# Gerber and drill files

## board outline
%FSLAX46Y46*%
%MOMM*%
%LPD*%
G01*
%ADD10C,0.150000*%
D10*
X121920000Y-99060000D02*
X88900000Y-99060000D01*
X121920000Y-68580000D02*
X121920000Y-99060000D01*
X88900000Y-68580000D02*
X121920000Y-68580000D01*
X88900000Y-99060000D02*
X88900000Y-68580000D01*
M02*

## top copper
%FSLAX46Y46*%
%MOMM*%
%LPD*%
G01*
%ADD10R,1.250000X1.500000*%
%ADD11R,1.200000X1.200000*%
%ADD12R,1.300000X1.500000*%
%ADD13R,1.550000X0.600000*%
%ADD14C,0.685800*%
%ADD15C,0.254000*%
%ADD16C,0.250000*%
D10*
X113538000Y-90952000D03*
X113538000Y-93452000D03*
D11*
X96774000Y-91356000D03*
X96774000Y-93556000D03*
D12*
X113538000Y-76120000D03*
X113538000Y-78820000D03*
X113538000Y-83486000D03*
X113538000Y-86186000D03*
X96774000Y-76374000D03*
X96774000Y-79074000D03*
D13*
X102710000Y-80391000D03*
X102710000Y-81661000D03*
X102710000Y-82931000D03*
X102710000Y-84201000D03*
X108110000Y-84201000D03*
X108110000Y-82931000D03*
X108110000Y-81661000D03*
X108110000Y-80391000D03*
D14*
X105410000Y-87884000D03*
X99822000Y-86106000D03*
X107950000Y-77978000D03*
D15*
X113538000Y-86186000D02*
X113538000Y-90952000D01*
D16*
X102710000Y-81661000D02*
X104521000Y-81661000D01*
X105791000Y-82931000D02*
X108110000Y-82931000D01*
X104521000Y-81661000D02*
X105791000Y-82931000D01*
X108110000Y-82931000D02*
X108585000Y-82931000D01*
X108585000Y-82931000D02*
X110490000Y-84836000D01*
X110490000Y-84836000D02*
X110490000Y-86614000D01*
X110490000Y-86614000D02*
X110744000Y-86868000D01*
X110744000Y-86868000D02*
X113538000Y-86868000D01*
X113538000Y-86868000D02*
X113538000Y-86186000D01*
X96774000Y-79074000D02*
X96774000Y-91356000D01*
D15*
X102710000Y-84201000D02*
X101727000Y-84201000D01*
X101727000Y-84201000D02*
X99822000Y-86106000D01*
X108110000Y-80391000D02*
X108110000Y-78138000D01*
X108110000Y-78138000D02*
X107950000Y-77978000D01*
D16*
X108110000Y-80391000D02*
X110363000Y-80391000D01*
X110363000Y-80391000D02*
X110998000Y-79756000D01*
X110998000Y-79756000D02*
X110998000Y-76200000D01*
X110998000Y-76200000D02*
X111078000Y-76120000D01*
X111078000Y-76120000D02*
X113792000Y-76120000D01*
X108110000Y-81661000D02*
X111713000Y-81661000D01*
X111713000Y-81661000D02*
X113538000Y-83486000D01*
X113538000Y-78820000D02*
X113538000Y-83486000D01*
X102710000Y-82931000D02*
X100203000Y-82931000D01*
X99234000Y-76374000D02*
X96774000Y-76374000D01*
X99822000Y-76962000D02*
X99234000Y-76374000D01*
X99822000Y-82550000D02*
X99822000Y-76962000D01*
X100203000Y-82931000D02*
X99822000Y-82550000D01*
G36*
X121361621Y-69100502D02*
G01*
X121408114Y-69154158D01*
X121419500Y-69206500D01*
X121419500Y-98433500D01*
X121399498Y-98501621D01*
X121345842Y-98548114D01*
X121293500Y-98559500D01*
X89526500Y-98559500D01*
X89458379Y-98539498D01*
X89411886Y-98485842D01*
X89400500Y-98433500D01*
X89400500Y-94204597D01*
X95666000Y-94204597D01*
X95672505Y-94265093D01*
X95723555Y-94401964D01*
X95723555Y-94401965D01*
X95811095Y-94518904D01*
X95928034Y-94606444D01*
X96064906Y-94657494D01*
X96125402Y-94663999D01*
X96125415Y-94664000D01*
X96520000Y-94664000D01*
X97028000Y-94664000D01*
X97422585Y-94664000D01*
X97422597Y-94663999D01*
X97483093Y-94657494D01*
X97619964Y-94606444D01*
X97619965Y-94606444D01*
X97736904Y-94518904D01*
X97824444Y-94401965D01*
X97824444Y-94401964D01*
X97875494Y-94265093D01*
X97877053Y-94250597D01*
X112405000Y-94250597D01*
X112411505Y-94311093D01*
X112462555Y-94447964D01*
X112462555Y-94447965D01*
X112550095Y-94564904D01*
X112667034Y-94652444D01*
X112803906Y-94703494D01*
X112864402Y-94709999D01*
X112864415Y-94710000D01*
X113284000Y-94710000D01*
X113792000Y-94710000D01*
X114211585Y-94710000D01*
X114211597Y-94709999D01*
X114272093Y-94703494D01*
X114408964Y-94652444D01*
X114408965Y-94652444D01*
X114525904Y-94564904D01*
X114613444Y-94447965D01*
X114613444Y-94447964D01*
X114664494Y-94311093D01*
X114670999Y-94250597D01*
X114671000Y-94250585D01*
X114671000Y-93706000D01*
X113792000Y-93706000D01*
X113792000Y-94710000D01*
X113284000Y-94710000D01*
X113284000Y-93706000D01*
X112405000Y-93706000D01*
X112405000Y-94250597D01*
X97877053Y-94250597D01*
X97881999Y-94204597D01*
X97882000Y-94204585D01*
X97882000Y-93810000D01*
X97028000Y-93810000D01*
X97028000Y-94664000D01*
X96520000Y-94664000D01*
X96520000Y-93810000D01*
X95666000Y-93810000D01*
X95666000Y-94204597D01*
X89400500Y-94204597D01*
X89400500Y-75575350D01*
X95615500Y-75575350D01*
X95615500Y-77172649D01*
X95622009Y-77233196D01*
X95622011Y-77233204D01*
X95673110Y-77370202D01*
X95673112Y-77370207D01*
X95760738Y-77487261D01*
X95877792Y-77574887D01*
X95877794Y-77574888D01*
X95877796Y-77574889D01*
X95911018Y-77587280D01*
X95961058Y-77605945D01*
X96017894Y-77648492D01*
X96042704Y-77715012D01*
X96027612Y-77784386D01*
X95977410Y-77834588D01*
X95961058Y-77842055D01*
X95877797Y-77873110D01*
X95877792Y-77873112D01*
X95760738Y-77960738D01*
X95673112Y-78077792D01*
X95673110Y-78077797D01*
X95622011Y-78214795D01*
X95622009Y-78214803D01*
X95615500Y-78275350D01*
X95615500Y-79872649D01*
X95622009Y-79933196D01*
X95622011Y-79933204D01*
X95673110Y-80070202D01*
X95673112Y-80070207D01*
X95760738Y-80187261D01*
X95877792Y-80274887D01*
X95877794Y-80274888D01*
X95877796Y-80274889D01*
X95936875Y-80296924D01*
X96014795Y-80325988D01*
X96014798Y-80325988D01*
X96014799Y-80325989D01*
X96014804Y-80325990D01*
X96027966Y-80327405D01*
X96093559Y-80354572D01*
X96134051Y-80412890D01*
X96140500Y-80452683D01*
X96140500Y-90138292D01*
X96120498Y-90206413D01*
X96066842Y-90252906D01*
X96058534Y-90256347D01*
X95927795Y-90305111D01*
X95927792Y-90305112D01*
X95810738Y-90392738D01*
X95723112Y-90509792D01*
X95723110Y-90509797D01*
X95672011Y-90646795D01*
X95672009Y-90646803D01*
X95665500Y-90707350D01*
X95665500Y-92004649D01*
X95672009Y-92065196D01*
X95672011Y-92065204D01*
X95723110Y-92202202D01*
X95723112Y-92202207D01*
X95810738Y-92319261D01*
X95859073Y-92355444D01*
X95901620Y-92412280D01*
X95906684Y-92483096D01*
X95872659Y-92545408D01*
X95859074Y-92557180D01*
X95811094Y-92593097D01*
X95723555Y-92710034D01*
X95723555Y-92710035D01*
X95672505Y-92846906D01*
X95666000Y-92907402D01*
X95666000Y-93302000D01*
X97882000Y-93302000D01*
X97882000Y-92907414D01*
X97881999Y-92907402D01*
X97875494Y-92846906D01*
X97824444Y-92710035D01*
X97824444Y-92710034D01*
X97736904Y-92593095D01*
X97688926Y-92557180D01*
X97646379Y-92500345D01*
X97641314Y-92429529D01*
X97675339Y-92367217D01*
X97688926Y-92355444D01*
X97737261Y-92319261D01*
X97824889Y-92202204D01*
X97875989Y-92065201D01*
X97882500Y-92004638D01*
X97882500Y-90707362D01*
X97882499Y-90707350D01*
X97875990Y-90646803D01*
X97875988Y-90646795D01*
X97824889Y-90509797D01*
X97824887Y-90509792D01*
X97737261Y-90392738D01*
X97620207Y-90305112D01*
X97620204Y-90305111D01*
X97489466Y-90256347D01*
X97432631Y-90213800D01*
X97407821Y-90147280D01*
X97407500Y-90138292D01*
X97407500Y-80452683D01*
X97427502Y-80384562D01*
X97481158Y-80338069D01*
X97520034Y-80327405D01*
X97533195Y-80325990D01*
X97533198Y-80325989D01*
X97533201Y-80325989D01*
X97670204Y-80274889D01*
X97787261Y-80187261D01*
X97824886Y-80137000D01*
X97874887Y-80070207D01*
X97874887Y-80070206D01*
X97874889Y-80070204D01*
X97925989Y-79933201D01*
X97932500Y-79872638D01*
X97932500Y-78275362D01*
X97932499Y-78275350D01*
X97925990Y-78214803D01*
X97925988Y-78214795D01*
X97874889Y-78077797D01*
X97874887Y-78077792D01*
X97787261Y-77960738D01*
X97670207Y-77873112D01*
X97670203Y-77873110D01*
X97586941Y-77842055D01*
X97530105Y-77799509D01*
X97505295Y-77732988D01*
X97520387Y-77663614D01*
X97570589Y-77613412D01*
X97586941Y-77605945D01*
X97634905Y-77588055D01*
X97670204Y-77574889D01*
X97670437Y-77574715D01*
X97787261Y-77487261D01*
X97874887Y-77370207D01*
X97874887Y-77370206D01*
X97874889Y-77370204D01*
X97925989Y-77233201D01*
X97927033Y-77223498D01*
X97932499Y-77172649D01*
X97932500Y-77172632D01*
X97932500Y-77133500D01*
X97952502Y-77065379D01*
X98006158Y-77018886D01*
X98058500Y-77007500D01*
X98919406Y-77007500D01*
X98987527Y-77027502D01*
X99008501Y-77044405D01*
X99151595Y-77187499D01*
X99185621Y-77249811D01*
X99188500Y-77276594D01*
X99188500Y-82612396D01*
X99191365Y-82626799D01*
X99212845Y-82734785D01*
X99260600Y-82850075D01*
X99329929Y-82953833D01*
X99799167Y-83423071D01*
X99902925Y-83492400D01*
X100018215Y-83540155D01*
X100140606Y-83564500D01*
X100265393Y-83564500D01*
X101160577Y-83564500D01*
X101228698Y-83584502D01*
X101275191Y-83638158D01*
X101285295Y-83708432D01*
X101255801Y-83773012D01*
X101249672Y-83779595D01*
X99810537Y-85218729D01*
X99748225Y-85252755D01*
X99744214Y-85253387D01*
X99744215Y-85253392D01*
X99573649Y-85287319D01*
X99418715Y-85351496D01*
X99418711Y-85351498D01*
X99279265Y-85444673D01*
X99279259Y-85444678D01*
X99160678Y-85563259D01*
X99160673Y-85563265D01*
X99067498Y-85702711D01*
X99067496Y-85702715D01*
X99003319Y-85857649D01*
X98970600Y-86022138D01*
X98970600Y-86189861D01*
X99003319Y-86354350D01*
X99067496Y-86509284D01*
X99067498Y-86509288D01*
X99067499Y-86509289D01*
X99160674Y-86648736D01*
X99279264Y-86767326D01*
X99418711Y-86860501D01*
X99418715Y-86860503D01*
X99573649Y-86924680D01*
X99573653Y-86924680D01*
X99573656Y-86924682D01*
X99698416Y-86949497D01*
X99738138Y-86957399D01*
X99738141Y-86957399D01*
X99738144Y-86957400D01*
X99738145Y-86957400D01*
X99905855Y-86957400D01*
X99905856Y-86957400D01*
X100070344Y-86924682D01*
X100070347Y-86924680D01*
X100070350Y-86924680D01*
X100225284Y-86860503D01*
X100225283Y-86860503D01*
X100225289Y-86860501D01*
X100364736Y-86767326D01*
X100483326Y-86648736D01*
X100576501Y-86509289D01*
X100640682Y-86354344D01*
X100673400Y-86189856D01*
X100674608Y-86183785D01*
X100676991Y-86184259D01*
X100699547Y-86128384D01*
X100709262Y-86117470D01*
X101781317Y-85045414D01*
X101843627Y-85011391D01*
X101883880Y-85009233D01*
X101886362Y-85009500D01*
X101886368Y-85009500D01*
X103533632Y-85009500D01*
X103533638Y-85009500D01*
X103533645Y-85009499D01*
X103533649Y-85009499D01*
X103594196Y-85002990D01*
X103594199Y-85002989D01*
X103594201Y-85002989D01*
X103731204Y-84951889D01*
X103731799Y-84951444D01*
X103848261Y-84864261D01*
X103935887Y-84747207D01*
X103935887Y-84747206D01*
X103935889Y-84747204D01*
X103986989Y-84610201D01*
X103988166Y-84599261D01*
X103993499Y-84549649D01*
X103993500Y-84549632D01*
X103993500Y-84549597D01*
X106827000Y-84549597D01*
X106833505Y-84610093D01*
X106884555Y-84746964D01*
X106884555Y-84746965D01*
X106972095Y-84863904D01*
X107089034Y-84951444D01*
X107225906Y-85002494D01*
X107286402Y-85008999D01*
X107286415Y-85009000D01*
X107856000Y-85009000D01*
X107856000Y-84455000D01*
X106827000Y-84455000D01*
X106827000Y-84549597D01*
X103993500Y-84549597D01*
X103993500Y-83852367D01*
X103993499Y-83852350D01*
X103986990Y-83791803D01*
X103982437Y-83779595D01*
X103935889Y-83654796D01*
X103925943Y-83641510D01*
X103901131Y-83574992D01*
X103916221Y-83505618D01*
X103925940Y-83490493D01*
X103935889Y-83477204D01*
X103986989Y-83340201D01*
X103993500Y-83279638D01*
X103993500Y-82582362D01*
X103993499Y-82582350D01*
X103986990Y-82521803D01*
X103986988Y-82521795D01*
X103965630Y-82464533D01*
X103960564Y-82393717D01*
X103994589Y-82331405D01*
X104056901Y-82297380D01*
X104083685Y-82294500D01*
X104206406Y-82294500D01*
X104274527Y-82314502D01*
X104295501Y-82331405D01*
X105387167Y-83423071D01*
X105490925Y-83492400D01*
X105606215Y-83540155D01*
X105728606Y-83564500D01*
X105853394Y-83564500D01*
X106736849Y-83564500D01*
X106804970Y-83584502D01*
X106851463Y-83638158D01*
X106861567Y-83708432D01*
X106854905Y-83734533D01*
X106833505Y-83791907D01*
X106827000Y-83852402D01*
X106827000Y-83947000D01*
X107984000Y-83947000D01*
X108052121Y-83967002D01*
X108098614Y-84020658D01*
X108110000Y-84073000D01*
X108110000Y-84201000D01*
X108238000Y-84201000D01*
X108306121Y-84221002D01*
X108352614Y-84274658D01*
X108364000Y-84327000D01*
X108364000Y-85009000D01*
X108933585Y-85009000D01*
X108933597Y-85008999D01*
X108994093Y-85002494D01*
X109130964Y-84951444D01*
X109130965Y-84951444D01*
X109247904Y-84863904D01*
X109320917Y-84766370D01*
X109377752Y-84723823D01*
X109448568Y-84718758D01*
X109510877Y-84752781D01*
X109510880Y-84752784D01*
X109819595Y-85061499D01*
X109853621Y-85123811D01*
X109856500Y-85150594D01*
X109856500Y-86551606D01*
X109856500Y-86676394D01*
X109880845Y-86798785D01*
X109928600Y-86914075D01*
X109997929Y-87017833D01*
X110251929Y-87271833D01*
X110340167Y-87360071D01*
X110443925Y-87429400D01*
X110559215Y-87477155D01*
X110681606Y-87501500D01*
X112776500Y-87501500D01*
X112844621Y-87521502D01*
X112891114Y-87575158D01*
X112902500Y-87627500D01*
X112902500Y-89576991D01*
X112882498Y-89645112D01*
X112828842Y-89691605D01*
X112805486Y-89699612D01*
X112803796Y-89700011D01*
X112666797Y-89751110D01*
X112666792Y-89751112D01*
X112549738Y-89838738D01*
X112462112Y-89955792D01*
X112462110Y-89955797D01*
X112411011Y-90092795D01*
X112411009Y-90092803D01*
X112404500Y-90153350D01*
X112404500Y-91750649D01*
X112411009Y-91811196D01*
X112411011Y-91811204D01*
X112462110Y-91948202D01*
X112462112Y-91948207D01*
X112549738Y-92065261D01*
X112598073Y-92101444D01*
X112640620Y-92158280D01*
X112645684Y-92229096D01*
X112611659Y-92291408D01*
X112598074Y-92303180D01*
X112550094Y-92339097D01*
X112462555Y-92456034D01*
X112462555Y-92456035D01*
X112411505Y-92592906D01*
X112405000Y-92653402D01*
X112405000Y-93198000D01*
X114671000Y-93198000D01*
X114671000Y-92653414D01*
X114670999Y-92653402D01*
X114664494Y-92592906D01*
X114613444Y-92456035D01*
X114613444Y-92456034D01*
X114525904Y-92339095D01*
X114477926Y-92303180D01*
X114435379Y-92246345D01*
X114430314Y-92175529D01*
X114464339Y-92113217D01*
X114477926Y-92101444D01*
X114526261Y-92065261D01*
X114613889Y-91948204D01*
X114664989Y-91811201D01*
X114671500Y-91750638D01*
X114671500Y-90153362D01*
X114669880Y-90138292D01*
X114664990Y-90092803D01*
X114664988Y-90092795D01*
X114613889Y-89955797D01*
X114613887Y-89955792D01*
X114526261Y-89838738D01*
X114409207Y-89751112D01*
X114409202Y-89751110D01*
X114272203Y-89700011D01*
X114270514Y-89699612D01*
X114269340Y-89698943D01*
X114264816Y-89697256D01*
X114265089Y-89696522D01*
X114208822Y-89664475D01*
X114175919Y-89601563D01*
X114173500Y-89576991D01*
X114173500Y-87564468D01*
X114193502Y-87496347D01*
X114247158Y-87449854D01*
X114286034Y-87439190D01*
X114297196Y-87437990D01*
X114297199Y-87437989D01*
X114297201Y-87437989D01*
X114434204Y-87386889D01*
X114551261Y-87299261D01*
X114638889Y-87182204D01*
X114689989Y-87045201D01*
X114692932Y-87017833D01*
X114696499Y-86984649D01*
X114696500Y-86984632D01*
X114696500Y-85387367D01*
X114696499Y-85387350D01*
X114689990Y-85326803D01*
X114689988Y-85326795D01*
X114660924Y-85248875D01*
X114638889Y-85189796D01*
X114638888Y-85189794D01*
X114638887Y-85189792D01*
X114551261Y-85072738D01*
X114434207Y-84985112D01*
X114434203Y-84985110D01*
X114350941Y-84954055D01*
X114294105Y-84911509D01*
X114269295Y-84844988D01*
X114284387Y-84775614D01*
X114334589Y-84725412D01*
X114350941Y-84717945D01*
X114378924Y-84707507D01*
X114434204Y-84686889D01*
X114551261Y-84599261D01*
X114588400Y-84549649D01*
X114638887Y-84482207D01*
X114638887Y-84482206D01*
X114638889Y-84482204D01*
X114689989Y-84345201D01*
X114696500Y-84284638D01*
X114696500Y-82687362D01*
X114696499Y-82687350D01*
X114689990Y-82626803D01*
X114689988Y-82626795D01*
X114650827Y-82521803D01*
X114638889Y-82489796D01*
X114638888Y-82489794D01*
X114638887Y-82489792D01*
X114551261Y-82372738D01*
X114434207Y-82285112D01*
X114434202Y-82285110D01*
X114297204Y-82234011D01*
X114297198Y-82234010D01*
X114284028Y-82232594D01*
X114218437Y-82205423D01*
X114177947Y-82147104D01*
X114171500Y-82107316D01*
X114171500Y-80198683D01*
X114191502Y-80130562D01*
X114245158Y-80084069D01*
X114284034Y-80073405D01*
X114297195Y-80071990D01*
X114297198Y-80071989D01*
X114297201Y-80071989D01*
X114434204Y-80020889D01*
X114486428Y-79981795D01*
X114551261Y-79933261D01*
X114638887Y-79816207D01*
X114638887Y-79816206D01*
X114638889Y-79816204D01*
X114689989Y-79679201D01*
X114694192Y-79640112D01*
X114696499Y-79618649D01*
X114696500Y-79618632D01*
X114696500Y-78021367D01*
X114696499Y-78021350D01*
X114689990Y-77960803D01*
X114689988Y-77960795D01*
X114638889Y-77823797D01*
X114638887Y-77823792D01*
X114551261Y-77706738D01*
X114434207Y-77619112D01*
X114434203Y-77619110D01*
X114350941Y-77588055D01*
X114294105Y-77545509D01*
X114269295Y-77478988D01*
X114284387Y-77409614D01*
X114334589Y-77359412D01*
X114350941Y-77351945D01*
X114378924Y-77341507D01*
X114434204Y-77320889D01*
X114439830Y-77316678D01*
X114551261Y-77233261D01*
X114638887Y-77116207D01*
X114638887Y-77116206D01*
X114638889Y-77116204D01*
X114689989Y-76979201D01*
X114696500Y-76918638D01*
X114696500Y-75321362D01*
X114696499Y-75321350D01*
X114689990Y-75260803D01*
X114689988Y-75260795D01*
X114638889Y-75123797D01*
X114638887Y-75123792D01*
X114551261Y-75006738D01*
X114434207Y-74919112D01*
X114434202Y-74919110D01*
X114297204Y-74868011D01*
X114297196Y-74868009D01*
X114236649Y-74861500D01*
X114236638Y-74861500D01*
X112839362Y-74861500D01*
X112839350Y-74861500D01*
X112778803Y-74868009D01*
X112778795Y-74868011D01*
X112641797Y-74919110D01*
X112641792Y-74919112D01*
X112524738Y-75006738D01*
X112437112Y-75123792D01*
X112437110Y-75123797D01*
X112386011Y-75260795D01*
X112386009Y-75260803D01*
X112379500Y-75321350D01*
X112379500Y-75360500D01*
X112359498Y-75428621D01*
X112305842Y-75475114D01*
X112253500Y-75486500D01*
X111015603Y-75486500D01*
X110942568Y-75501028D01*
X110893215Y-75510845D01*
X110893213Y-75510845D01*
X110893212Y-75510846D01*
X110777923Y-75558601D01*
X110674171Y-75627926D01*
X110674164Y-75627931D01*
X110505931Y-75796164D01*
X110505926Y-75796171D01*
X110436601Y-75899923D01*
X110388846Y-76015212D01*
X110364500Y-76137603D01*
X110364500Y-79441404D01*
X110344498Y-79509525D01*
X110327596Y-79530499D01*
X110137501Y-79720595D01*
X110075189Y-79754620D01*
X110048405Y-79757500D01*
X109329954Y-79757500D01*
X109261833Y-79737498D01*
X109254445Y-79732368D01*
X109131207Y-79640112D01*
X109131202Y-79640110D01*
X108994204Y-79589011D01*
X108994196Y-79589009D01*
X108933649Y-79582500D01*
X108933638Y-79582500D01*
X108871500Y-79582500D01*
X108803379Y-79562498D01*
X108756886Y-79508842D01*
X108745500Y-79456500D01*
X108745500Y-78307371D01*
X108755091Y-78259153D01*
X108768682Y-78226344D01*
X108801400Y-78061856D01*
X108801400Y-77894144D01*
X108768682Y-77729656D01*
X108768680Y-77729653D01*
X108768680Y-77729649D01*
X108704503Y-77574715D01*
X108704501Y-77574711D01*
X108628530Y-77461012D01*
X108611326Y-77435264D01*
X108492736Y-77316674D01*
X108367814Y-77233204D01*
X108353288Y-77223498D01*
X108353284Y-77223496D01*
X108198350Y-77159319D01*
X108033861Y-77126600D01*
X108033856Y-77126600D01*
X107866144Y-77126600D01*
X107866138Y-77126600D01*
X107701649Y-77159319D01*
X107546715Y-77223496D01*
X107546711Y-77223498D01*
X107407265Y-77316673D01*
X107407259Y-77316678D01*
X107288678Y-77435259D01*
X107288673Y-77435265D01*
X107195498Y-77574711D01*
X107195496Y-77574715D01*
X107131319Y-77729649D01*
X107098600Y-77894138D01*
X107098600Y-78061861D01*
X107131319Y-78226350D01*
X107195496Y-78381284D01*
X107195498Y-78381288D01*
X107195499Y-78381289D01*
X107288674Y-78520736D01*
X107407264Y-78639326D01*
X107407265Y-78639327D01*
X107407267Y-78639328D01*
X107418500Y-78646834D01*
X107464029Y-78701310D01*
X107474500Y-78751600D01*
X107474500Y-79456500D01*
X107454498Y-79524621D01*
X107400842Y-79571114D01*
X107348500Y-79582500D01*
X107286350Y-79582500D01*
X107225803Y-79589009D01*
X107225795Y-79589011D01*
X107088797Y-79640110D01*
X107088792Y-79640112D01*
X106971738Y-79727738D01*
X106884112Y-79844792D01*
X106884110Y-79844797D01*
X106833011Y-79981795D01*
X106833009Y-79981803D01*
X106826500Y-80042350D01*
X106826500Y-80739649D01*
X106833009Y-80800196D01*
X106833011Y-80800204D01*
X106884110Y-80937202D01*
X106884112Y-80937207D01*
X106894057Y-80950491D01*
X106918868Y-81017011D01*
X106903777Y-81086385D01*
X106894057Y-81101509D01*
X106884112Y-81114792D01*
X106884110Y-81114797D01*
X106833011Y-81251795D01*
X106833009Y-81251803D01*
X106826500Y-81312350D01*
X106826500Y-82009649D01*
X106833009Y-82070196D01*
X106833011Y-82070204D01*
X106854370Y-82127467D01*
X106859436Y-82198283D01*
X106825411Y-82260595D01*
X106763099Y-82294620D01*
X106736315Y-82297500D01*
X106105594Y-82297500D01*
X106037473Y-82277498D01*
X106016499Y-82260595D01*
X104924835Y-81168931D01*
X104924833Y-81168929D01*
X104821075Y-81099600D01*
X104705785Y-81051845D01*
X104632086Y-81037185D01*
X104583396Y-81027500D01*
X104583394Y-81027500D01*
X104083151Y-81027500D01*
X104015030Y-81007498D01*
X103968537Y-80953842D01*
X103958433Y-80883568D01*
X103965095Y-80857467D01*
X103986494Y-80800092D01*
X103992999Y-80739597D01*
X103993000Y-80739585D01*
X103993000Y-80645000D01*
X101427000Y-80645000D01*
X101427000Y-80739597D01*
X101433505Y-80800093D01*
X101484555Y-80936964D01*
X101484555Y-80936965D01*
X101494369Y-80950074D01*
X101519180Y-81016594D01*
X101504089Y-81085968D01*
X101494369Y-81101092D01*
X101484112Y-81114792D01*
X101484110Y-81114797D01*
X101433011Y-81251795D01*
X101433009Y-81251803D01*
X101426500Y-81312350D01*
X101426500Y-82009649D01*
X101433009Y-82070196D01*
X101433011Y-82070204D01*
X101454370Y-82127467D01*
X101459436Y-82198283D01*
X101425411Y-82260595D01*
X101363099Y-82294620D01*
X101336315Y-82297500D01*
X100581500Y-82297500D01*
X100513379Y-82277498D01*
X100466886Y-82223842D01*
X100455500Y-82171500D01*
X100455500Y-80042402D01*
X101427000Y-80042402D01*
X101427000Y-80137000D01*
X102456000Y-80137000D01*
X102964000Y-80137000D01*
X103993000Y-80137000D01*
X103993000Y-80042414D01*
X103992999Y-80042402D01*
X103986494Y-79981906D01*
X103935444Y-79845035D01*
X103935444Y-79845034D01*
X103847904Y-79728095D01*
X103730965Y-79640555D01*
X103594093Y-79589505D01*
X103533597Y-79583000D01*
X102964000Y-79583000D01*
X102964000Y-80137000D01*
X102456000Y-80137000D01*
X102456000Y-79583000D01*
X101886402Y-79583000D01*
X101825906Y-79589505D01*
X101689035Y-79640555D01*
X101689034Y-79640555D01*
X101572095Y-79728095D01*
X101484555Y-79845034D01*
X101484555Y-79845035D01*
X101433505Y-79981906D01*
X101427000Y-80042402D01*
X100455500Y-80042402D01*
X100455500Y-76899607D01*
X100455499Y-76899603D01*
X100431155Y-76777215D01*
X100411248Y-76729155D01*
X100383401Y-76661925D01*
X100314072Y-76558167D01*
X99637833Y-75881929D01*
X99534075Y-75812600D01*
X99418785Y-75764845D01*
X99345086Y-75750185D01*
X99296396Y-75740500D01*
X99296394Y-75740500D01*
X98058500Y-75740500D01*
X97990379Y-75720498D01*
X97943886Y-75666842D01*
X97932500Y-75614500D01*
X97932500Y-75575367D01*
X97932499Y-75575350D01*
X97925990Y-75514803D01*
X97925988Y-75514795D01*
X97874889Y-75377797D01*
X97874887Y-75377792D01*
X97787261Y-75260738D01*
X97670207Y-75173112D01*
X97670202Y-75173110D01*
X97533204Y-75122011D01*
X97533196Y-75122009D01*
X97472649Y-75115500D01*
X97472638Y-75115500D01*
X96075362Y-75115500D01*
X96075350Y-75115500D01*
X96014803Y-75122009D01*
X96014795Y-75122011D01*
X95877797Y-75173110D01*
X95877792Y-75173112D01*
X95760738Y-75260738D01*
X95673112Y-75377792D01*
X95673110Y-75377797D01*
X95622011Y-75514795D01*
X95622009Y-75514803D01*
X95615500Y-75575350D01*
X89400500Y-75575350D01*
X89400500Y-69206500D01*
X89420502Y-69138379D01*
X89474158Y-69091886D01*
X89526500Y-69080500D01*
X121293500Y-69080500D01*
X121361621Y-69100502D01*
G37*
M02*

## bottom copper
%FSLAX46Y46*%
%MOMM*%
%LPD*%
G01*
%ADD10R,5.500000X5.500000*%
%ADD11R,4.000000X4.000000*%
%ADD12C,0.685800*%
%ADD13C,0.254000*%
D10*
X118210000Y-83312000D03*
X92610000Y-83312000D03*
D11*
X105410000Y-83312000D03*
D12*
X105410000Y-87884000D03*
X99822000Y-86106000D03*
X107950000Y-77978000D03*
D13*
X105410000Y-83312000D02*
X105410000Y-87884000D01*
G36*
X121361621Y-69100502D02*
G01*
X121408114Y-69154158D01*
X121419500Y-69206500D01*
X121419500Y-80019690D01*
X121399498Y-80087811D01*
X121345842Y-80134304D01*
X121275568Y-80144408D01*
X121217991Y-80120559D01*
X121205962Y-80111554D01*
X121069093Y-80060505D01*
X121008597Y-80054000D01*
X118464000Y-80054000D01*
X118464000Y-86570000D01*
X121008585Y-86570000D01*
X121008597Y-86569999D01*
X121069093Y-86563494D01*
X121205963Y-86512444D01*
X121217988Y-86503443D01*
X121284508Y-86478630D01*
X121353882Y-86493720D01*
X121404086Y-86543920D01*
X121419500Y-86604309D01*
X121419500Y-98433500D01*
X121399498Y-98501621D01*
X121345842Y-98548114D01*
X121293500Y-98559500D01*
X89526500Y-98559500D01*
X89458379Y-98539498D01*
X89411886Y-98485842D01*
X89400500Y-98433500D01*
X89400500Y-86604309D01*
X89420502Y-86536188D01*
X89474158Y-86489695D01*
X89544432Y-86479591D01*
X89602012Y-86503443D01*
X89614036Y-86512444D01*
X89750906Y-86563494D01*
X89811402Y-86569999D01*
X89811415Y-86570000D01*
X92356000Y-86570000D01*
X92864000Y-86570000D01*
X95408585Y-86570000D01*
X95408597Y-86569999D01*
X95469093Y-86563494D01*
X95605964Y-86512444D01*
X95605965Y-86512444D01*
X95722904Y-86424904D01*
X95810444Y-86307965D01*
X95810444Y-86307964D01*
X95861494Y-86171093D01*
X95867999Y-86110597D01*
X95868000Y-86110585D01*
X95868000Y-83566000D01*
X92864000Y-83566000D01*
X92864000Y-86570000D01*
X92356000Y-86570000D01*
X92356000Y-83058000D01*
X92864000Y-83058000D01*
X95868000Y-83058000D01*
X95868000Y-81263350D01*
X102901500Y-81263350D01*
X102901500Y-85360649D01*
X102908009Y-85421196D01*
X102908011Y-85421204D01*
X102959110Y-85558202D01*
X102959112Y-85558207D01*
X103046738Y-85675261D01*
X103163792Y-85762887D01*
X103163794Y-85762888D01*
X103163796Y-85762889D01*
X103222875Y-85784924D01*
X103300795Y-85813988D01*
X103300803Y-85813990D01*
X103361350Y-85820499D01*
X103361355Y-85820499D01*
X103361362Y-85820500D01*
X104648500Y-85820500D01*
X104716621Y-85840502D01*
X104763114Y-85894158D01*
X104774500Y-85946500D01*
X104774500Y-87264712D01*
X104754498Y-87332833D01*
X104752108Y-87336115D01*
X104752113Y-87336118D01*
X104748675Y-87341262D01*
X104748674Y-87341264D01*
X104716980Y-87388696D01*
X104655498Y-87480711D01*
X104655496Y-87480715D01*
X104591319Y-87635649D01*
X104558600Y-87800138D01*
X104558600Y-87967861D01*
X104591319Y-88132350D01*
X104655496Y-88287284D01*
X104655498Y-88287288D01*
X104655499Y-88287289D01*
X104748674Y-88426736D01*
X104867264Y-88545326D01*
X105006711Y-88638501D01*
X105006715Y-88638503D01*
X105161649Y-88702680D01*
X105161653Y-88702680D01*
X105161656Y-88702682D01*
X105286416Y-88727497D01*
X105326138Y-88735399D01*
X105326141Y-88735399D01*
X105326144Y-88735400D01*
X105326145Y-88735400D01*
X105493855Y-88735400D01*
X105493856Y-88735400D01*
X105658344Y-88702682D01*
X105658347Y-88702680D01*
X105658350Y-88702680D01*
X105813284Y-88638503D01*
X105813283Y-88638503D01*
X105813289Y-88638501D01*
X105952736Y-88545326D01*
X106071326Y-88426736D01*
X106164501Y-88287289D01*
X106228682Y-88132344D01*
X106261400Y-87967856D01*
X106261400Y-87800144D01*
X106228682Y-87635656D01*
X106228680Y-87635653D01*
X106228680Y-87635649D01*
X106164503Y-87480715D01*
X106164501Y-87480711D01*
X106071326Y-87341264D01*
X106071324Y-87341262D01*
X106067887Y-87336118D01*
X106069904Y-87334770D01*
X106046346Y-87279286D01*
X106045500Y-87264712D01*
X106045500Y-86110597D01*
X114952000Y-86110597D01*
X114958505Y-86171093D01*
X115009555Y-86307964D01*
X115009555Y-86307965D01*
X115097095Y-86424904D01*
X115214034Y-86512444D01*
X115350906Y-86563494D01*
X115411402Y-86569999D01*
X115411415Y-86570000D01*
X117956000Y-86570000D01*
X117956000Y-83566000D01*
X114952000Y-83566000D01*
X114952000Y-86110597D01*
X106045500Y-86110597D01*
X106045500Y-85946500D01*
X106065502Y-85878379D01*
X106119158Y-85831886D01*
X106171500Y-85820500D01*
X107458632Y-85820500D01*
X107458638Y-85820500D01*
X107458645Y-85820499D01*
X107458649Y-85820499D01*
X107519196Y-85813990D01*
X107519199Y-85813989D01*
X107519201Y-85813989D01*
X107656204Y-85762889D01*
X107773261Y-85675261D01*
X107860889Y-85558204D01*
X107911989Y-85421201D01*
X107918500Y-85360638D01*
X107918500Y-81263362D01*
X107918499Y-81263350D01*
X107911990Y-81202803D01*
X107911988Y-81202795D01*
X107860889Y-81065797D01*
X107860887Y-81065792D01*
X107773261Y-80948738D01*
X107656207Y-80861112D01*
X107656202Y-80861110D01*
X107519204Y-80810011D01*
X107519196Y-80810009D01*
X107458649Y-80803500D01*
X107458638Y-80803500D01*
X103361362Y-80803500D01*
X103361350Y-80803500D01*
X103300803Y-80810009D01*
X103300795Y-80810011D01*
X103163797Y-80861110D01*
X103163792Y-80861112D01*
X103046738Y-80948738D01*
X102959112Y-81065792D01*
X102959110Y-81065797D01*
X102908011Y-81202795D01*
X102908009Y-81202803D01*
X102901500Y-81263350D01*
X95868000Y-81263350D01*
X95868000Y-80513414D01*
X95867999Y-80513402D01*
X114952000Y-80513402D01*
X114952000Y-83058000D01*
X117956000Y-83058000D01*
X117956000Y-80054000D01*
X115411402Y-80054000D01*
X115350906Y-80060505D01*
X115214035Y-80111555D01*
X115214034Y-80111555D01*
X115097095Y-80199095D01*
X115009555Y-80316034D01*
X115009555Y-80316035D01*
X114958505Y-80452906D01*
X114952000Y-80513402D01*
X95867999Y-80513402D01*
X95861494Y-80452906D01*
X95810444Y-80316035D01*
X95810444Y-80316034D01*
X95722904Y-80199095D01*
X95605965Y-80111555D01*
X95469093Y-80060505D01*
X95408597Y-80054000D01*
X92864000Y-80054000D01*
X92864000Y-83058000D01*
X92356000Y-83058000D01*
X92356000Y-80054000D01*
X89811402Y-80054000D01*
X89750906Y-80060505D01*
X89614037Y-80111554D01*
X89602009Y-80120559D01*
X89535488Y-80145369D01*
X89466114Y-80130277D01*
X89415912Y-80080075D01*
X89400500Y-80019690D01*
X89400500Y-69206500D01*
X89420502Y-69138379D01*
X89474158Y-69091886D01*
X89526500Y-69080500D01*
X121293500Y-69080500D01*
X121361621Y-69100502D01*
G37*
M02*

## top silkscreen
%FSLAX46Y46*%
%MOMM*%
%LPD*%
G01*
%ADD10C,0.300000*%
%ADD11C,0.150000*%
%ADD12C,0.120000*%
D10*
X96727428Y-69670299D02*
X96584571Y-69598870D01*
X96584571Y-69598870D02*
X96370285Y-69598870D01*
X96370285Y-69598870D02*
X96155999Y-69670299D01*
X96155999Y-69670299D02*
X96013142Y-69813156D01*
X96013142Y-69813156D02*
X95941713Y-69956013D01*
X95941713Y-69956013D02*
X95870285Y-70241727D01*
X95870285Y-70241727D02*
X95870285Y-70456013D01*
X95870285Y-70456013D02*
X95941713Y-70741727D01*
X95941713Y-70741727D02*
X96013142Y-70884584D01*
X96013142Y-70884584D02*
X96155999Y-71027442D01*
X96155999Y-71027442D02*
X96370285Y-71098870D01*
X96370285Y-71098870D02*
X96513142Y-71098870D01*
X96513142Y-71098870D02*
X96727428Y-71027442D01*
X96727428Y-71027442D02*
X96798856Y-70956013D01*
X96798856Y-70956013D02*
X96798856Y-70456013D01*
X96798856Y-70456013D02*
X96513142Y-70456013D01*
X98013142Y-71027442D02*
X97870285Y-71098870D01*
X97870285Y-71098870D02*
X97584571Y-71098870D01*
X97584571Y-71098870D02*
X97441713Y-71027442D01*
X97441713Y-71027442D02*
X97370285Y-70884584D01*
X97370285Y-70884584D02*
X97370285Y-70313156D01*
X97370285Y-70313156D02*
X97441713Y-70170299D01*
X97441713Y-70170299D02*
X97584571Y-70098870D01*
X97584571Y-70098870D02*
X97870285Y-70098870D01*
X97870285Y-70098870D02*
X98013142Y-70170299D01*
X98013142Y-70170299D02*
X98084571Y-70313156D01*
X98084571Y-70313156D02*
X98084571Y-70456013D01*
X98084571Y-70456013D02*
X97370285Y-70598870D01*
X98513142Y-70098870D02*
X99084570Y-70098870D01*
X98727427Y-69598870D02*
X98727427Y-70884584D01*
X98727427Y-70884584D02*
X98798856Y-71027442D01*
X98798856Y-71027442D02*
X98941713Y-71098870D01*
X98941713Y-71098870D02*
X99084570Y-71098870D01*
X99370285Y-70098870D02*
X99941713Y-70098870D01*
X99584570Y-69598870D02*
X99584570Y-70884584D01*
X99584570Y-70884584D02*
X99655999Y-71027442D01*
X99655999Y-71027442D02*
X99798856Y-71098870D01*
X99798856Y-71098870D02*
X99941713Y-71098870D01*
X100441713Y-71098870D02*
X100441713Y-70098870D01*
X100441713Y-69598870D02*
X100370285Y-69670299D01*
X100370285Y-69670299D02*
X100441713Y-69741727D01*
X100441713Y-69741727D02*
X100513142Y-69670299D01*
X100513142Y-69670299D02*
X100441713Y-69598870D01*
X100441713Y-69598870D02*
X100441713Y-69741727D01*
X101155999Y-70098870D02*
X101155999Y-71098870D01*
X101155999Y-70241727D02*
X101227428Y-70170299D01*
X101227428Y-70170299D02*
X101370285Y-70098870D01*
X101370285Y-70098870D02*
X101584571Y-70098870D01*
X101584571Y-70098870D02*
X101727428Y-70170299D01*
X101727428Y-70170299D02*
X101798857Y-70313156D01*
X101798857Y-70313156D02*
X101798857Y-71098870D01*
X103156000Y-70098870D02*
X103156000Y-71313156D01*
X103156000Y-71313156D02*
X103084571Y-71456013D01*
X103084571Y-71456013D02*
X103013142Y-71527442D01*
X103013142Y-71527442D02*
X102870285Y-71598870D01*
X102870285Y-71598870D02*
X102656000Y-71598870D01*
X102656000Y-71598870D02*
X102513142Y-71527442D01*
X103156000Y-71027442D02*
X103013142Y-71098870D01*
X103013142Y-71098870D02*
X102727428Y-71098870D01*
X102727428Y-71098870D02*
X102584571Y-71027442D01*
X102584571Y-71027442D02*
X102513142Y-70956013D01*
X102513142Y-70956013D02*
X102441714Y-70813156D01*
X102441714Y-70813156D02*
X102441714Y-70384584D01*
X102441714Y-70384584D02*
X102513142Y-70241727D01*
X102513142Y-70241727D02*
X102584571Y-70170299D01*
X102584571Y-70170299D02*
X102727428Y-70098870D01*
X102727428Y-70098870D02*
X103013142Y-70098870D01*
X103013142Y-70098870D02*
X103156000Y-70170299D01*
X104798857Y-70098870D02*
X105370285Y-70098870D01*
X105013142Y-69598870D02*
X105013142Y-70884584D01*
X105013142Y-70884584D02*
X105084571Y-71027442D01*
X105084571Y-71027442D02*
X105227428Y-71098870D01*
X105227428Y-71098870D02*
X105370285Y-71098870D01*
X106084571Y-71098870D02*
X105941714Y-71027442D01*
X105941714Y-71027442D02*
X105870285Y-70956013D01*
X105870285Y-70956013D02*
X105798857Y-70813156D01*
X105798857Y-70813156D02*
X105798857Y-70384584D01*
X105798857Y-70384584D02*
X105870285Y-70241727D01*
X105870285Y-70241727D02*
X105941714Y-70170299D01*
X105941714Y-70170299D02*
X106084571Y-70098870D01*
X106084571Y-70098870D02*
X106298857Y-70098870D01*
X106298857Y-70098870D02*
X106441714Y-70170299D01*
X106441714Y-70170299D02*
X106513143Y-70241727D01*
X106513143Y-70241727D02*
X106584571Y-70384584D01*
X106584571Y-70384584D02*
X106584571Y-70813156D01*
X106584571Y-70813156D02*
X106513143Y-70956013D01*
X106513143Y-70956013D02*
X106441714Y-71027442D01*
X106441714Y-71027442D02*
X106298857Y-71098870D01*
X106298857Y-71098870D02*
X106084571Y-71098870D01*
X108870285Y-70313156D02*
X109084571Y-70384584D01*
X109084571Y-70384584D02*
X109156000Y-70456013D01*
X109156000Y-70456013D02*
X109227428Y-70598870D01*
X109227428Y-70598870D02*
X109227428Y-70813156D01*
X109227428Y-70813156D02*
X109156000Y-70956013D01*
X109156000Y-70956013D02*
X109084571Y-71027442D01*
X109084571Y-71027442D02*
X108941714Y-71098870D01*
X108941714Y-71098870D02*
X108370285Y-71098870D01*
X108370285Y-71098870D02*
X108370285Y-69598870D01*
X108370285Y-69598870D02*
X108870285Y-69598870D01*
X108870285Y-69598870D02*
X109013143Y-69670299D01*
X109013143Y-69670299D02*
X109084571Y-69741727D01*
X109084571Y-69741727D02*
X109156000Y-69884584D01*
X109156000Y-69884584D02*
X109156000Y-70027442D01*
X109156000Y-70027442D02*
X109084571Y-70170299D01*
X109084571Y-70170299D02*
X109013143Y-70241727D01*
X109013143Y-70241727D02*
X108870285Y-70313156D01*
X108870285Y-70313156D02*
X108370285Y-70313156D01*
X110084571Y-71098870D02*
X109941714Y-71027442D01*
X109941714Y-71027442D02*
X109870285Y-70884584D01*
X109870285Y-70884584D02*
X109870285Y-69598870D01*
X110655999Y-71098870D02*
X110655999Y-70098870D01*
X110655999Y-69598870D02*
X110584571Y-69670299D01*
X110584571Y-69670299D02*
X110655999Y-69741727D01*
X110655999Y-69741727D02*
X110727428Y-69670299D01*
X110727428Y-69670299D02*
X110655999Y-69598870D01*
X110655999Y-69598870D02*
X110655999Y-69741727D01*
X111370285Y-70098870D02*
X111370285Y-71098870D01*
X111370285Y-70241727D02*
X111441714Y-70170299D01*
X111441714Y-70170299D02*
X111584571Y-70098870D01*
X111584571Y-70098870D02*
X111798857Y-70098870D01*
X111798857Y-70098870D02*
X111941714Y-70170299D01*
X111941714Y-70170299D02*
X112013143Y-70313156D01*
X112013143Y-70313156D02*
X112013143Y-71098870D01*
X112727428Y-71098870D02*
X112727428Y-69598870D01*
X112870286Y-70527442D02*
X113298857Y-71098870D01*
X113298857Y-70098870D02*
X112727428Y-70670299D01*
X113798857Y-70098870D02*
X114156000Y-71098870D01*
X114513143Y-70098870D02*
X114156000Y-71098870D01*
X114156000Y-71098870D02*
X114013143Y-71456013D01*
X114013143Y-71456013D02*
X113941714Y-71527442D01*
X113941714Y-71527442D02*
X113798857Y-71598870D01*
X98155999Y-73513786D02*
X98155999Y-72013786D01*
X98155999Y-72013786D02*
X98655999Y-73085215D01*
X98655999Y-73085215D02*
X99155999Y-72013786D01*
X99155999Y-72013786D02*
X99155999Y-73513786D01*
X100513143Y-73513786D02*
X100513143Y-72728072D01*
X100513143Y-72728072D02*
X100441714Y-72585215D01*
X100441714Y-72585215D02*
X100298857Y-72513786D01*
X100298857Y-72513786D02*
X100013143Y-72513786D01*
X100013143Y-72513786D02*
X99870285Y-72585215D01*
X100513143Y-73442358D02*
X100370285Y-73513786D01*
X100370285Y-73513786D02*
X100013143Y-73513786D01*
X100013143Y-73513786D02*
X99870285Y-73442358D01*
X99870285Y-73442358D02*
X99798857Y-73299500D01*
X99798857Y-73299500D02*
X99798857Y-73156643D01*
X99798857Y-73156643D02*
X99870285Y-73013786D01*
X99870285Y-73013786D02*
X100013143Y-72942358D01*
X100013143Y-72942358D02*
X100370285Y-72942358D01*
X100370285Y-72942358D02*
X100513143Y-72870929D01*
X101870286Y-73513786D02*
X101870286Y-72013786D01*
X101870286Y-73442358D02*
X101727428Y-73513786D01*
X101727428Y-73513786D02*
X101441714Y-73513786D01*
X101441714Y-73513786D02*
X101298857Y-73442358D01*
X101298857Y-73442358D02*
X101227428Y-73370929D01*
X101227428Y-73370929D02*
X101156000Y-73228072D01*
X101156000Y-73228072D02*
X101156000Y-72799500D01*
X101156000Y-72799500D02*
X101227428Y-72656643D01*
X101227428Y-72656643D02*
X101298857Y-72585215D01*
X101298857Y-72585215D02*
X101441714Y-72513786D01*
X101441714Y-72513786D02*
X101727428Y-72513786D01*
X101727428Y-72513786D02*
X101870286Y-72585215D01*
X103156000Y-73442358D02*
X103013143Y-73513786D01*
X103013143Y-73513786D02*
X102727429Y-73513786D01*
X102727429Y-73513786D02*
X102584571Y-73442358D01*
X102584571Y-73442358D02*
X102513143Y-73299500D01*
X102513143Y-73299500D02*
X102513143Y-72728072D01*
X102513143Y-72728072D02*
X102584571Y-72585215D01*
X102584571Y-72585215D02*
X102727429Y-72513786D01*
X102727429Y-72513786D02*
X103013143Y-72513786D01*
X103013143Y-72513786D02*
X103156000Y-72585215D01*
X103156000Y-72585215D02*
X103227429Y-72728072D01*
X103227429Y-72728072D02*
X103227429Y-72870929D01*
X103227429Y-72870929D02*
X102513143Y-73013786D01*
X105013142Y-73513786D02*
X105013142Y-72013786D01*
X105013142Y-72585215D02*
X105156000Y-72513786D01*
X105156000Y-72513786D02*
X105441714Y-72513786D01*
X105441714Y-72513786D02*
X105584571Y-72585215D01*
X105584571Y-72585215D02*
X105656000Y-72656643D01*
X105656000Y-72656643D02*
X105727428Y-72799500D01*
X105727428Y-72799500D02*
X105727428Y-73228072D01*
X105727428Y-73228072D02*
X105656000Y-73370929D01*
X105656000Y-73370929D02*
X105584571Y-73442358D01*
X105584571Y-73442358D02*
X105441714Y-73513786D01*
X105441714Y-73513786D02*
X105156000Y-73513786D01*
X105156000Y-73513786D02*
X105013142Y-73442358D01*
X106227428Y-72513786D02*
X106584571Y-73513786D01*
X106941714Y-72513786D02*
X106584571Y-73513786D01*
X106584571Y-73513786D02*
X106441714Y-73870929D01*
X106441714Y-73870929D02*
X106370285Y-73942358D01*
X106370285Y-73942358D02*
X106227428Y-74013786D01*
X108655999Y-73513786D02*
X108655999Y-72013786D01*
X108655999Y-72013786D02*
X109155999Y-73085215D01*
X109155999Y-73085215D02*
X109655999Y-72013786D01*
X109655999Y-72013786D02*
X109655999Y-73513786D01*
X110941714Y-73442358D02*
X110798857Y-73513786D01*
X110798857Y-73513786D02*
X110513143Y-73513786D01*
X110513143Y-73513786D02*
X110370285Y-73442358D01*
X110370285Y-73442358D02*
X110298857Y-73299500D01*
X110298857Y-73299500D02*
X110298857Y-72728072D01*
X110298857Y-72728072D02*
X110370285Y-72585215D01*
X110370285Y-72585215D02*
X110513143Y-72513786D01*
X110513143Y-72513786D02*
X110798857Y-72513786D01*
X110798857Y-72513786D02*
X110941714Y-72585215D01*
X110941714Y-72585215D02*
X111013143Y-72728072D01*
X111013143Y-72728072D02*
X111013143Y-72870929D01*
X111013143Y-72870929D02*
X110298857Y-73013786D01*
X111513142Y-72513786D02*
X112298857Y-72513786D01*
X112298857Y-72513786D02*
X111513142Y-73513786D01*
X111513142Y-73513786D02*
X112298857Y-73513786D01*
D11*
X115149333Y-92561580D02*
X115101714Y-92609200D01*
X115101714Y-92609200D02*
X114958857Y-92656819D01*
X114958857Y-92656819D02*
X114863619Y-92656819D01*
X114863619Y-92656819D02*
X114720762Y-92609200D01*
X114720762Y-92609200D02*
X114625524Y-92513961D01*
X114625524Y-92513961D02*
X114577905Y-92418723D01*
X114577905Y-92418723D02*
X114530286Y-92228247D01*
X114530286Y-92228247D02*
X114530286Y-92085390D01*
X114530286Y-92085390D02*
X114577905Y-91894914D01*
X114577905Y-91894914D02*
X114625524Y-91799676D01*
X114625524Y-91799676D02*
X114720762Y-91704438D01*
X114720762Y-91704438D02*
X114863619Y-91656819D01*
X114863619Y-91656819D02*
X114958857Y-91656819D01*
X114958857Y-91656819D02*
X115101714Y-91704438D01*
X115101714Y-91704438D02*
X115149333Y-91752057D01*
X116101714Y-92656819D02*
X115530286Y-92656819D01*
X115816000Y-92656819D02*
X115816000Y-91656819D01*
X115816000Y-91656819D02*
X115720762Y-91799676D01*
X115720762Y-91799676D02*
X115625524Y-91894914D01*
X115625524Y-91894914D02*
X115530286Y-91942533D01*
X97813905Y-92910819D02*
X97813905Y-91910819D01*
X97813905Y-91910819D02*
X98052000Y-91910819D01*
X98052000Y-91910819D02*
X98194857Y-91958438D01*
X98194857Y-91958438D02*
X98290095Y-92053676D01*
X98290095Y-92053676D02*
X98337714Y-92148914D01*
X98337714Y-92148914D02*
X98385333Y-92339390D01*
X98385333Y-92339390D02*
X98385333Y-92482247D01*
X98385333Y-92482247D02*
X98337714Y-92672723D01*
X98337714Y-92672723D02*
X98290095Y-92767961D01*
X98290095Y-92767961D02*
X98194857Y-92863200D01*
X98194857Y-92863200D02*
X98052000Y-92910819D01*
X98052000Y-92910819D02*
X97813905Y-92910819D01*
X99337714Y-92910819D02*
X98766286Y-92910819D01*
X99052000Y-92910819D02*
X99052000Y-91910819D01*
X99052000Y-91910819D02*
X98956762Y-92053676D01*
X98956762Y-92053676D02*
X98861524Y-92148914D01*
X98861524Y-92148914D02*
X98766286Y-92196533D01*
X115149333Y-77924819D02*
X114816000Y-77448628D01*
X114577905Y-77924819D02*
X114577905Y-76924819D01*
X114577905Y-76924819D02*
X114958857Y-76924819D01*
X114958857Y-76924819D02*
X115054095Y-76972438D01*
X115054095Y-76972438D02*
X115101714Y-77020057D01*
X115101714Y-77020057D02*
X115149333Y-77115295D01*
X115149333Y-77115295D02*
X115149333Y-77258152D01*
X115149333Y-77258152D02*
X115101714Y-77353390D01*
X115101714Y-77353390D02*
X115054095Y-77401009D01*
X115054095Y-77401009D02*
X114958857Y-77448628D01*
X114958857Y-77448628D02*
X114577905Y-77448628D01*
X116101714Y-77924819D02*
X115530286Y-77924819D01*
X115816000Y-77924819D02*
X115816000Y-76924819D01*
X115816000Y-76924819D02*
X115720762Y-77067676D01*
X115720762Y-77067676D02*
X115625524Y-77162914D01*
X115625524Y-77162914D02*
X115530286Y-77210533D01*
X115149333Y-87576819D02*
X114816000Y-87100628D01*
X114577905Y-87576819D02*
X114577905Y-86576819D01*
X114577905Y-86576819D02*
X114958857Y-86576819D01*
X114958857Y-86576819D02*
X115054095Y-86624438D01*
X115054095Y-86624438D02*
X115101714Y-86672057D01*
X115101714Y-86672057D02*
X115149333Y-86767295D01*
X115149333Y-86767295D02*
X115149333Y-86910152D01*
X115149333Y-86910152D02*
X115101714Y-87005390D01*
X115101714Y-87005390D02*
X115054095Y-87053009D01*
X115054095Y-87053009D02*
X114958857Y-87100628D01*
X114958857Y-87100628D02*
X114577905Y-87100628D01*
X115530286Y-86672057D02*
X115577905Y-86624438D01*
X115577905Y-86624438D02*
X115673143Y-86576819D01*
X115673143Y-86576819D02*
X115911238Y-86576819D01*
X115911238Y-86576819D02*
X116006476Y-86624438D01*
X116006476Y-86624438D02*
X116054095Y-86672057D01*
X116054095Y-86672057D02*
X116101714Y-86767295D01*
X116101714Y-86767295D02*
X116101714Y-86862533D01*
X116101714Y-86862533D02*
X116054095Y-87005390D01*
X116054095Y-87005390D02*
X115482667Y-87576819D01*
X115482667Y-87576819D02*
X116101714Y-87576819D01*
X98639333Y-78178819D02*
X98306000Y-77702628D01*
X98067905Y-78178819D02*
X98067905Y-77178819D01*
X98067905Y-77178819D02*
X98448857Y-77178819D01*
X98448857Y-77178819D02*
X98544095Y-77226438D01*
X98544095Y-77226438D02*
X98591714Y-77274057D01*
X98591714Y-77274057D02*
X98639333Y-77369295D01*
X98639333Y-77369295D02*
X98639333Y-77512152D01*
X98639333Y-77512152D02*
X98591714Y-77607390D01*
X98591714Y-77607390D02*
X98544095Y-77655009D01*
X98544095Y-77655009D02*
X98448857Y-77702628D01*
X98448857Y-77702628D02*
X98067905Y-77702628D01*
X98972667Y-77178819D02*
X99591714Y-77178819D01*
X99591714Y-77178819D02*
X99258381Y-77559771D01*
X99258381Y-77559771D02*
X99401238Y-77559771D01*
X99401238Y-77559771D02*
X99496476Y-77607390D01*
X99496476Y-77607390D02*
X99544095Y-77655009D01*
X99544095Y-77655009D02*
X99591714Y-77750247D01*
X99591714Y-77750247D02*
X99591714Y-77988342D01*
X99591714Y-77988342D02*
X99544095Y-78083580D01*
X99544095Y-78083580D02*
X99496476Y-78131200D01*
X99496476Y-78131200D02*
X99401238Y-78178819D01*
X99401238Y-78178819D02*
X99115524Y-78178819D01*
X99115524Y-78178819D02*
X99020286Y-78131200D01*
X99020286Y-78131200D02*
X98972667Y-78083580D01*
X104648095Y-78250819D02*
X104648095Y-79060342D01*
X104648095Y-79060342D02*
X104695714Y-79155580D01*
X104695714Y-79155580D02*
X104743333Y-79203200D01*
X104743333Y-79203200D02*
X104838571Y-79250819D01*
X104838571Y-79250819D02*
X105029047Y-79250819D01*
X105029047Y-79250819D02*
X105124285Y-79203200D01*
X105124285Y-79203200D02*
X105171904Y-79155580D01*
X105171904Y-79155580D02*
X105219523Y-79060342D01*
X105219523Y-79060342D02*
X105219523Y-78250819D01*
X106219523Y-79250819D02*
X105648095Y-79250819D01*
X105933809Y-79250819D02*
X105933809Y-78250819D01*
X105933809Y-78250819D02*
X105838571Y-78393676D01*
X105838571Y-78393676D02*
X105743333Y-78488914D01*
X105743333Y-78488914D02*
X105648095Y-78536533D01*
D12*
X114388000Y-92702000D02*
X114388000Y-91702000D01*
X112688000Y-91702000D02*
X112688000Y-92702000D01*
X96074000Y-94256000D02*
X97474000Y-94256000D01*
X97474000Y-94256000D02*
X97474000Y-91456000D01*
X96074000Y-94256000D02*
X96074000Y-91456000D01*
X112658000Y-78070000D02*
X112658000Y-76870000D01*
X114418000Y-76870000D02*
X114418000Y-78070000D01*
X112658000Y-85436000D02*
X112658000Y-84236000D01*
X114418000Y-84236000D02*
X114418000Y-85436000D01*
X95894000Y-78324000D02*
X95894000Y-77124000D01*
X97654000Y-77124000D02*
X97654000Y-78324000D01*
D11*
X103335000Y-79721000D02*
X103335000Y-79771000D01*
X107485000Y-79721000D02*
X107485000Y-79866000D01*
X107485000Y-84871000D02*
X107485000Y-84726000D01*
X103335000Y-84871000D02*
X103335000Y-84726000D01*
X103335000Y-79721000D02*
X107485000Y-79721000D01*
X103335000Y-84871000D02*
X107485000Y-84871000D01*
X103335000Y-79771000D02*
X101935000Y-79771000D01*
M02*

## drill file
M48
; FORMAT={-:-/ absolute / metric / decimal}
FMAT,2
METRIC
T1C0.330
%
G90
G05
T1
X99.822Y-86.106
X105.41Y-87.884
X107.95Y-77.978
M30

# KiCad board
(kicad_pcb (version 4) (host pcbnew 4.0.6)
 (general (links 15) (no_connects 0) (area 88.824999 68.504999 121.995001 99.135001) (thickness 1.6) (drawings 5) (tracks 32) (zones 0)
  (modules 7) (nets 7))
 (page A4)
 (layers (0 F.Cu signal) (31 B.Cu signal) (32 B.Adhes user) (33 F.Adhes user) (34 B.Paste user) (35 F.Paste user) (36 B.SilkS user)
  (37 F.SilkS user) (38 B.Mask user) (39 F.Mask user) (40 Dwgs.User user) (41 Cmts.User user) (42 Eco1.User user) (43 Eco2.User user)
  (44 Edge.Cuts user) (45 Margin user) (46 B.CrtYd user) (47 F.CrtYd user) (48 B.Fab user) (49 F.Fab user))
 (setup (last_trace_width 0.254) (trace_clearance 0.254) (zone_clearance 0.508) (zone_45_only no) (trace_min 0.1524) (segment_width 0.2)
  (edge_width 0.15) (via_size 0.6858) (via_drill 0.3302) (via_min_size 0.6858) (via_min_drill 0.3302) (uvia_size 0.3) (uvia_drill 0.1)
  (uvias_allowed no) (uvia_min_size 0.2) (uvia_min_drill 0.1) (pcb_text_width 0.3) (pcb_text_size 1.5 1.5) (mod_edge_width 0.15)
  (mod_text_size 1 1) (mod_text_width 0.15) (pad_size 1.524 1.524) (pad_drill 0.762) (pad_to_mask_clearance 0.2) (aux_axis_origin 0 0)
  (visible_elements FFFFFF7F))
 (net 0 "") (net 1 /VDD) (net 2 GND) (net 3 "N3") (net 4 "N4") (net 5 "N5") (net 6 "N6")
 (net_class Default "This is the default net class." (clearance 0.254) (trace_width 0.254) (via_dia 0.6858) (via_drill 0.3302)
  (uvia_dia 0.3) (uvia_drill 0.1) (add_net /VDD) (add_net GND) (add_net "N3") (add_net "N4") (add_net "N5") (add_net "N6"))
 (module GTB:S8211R (layer B.Cu) (at 105.41 83.312)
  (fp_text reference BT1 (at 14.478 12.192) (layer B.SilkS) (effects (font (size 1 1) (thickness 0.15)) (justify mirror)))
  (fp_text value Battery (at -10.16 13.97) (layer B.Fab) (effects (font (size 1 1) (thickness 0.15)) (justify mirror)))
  (pad 1 smd rect (at 12.8 0) (size 5.5 5.5) (layers B.Cu B.Paste B.Mask) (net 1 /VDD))
  (pad 1 smd rect (at -12.8 0) (size 5.5 5.5) (layers B.Cu B.Paste B.Mask) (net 1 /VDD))
  (pad 2 smd rect (at 0 0) (size 4 4) (layers B.Cu B.Paste B.Mask) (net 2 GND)))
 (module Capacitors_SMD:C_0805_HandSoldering (layer F.Cu) (at 113.538 92.202 270)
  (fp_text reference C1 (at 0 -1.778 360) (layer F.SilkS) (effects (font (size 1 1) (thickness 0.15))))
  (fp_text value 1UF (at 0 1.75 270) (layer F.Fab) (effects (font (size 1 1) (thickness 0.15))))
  (fp_line (start 0.5 -0.85) (end -0.5 -0.85) (layer F.SilkS) (width 0.12))
  (fp_line (start -0.5 0.85) (end 0.5 0.85) (layer F.SilkS) (width 0.12))
  (pad 1 smd rect (at -1.25 0 270) (size 1.5 1.25) (layers F.Cu F.Paste F.Mask) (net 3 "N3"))
  (pad 2 smd rect (at 1.25 0 270) (size 1.5 1.25) (layers F.Cu F.Paste F.Mask) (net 2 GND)))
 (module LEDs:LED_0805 (layer F.Cu) (at 96.774 92.456 90)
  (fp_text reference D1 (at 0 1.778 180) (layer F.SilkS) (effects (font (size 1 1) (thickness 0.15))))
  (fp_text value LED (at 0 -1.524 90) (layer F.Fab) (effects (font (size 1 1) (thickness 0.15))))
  (fp_line (start -1.8 -0.7) (end -1.8 0.7) (layer F.SilkS) (width 0.12))
  (fp_line (start -1.8 0.7) (end 1 0.7) (layer F.SilkS) (width 0.12))
  (fp_line (start -1.8 -0.7) (end 1 -0.7) (layer F.SilkS) (width 0.12))
  (pad 2 smd rect (at 1.1 0 270) (size 1.2 1.2) (layers F.Cu F.Paste F.Mask) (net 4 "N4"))
  (pad 1 smd rect (at -1.1 0 270) (size 1.2 1.2) (layers F.Cu F.Paste F.Mask) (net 2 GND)))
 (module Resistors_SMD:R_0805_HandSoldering (layer F.Cu) (at 113.538 77.47 270)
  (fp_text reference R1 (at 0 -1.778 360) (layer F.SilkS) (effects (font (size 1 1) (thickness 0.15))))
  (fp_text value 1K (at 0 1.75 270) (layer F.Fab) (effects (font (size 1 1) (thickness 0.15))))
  (fp_line (start 0.6 0.88) (end -0.6 0.88) (layer F.SilkS) (width 0.12))
  (fp_line (start -0.6 -0.88) (end 0.6 -0.88) (layer F.SilkS) (width 0.12))
  (pad 1 smd rect (at -1.35 0 270) (size 1.5 1.3) (layers F.Cu F.Paste F.Mask) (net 1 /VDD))
  (pad 2 smd rect (at 1.35 0 270) (size 1.5 1.3) (layers F.Cu F.Paste F.Mask) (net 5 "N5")))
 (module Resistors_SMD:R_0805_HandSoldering (layer F.Cu) (at 113.538 84.836 270)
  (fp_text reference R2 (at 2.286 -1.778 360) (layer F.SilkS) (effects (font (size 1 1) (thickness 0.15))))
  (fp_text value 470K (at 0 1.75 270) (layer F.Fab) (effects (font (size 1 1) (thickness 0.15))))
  (fp_line (start 0.6 0.88) (end -0.6 0.88) (layer F.SilkS) (width 0.12))
  (fp_line (start -0.6 -0.88) (end 0.6 -0.88) (layer F.SilkS) (width 0.12))
  (pad 1 smd rect (at -1.35 0 270) (size 1.5 1.3) (layers F.Cu F.Paste F.Mask) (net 5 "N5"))
  (pad 2 smd rect (at 1.35 0 270) (size 1.5 1.3) (layers F.Cu F.Paste F.Mask) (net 3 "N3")))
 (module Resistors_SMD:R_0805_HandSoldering (layer F.Cu) (at 96.774 77.724 270)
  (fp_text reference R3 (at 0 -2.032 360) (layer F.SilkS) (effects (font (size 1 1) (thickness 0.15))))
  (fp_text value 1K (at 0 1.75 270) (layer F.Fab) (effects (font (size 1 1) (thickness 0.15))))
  (fp_line (start 0.6 0.88) (end -0.6 0.88) (layer F.SilkS) (width 0.12))
  (fp_line (start -0.6 -0.88) (end 0.6 -0.88) (layer F.SilkS) (width 0.12))
  (pad 1 smd rect (at -1.35 0 270) (size 1.5 1.3) (layers F.Cu F.Paste F.Mask) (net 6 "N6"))
  (pad 2 smd rect (at 1.35 0 270) (size 1.5 1.3) (layers F.Cu F.Paste F.Mask) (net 4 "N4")))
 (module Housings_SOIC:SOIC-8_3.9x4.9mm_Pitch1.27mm (layer F.Cu) (at 105.41 82.296)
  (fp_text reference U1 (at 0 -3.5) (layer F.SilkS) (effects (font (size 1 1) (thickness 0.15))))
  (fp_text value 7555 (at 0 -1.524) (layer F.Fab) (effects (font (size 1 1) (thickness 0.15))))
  (fp_line (start -2.075 -2.575) (end -2.075 -2.525) (layer F.SilkS) (width 0.15))
  (fp_line (start 2.075 -2.575) (end 2.075 -2.43) (layer F.SilkS) (width 0.15))
  (fp_line (start 2.075 2.575) (end 2.075 2.43) (layer F.SilkS) (width 0.15))
  (fp_line (start -2.075 2.575) (end -2.075 2.43) (layer F.SilkS) (width 0.15))
  (fp_line (start -2.075 -2.575) (end 2.075 -2.575) (layer F.SilkS) (width 0.15))
  (fp_line (start -2.075 2.575) (end 2.075 2.575) (layer F.SilkS) (width 0.15))
  (fp_line (start -2.075 -2.525) (end -3.475 -2.525) (layer F.SilkS) (width 0.15))
  (pad 1 smd rect (at -2.7 -1.905) (size 1.55 0.6) (layers F.Cu F.Paste F.Mask) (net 2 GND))
  (pad 2 smd rect (at -2.7 -0.635) (size 1.55 0.6) (layers F.Cu F.Paste F.Mask) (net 3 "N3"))
  (pad 3 smd rect (at -2.7 0.635) (size 1.55 0.6) (layers F.Cu F.Paste F.Mask) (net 6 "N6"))
  (pad 4 smd rect (at -2.7 1.905) (size 1.55 0.6) (layers F.Cu F.Paste F.Mask) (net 1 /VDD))
  (pad 5 smd rect (at 2.7 1.905) (size 1.55 0.6) (layers F.Cu F.Paste F.Mask) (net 2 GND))
  (pad 6 smd rect (at 2.7 0.635) (size 1.55 0.6) (layers F.Cu F.Paste F.Mask) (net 3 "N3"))
  (pad 7 smd rect (at 2.7 -0.635) (size 1.55 0.6) (layers F.Cu F.Paste F.Mask) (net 5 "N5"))
  (pad 8 smd rect (at 2.7 -1.905) (size 1.55 0.6) (layers F.Cu F.Paste F.Mask) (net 1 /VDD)))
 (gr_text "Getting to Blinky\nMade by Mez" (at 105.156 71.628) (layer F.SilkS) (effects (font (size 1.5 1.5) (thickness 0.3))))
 (gr_line (start 121.92 99.06) (end 88.9 99.06) (angle 90) (layer Edge.Cuts) (width 0.15))
 (gr_line (start 121.92 68.58) (end 121.92 99.06) (angle 90) (layer Edge.Cuts) (width 0.15))
 (gr_line (start 88.9 68.58) (end 121.92 68.58) (angle 90) (layer Edge.Cuts) (width 0.15))
 (gr_line (start 88.9 99.06) (end 88.9 68.58) (angle 90) (layer Edge.Cuts) (width 0.15))
 (segment (start 113.538 86.186) (end 113.538 90.952) (width 0.254) (layer F.Cu) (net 3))
 (segment (start 102.71 81.661) (end 104.521 81.661) (width 0.25) (layer F.Cu) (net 3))
 (segment (start 105.791 82.931) (end 108.11 82.931) (width 0.25) (layer F.Cu) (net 3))
 (segment (start 104.521 81.661) (end 105.791 82.931) (width 0.25) (layer F.Cu) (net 3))
 (segment (start 108.11 82.931) (end 108.585 82.931) (width 0.25) (layer F.Cu) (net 3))
 (segment (start 108.585 82.931) (end 110.49 84.836) (width 0.25) (layer F.Cu) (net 3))
 (segment (start 110.49 84.836) (end 110.49 86.614) (width 0.25) (layer F.Cu) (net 3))
 (segment (start 110.49 86.614) (end 110.744 86.868) (width 0.25) (layer F.Cu) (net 3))
 (segment (start 110.744 86.868) (end 113.538 86.868) (width 0.25) (layer F.Cu) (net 3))
 (segment (start 113.538 86.868) (end 113.538 86.186) (width 0.25) (layer F.Cu) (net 3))
 (segment (start 105.41 83.312) (end 105.41 87.884) (width 0.254) (layer B.Cu) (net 2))
 (via (at 105.41 87.884) (size 0.6858) (drill 0.3302) (layers F.Cu B.Cu) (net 2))
 (segment (start 96.774 79.074) (end 96.774 91.356) (width 0.25) (layer F.Cu) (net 4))
 (segment (start 102.71 84.201) (end 101.727 84.201) (width 0.254) (layer F.Cu) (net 1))
 (via (at 99.822 86.106) (size 0.6858) (drill 0.3302) (layers F.Cu B.Cu) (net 1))
 (segment (start 101.727 84.201) (end 99.822 86.106) (width 0.254) (layer F.Cu) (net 1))
 (segment (start 108.11 80.391) (end 108.11 78.138) (width 0.254) (layer F.Cu) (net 1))
 (via (at 107.95 77.978) (size 0.6858) (drill 0.3302) (layers F.Cu B.Cu) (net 1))
 (segment (start 108.11 78.138) (end 107.95 77.978) (width 0.254) (layer F.Cu) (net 1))
 (segment (start 108.11 80.391) (end 110.363 80.391) (width 0.25) (layer F.Cu) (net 1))
 (segment (start 110.363 80.391) (end 110.998 79.756) (width 0.25) (layer F.Cu) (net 1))
 (segment (start 110.998 79.756) (end 110.998 76.2) (width 0.25) (layer F.Cu) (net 1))
 (segment (start 110.998 76.2) (end 111.078 76.12) (width 0.25) (layer F.Cu) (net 1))
 (segment (start 111.078 76.12) (end 113.792 76.12) (width 0.25) (layer F.Cu) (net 1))
 (segment (start 108.11 81.661) (end 111.713 81.661) (width 0.25) (layer F.Cu) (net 5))
 (segment (start 111.713 81.661) (end 113.538 83.486) (width 0.25) (layer F.Cu) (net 5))
 (segment (start 113.538 78.82) (end 113.538 83.486) (width 0.25) (layer F.Cu) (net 5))
 (segment (start 102.71 82.931) (end 100.203 82.931) (width 0.25) (layer F.Cu) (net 6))
 (segment (start 99.234 76.374) (end 96.774 76.374) (width 0.25) (layer F.Cu) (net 6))
 (segment (start 99.822 76.962) (end 99.234 76.374) (width 0.25) (layer F.Cu) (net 6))
 (segment (start 99.822 82.55) (end 99.822 76.962) (width 0.25) (layer F.Cu) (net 6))
 (segment (start 100.203 82.931) (end 99.822 82.55) (width 0.25) (layer F.Cu) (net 6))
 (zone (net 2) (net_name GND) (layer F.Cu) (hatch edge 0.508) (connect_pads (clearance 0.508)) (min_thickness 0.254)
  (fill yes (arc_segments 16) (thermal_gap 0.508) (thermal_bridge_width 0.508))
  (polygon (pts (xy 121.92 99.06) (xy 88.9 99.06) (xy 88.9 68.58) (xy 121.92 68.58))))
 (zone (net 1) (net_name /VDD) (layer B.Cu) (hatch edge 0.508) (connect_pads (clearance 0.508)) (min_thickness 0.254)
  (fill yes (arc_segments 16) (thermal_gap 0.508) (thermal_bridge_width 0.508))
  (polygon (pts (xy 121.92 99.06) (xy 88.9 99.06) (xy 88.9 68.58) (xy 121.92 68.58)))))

